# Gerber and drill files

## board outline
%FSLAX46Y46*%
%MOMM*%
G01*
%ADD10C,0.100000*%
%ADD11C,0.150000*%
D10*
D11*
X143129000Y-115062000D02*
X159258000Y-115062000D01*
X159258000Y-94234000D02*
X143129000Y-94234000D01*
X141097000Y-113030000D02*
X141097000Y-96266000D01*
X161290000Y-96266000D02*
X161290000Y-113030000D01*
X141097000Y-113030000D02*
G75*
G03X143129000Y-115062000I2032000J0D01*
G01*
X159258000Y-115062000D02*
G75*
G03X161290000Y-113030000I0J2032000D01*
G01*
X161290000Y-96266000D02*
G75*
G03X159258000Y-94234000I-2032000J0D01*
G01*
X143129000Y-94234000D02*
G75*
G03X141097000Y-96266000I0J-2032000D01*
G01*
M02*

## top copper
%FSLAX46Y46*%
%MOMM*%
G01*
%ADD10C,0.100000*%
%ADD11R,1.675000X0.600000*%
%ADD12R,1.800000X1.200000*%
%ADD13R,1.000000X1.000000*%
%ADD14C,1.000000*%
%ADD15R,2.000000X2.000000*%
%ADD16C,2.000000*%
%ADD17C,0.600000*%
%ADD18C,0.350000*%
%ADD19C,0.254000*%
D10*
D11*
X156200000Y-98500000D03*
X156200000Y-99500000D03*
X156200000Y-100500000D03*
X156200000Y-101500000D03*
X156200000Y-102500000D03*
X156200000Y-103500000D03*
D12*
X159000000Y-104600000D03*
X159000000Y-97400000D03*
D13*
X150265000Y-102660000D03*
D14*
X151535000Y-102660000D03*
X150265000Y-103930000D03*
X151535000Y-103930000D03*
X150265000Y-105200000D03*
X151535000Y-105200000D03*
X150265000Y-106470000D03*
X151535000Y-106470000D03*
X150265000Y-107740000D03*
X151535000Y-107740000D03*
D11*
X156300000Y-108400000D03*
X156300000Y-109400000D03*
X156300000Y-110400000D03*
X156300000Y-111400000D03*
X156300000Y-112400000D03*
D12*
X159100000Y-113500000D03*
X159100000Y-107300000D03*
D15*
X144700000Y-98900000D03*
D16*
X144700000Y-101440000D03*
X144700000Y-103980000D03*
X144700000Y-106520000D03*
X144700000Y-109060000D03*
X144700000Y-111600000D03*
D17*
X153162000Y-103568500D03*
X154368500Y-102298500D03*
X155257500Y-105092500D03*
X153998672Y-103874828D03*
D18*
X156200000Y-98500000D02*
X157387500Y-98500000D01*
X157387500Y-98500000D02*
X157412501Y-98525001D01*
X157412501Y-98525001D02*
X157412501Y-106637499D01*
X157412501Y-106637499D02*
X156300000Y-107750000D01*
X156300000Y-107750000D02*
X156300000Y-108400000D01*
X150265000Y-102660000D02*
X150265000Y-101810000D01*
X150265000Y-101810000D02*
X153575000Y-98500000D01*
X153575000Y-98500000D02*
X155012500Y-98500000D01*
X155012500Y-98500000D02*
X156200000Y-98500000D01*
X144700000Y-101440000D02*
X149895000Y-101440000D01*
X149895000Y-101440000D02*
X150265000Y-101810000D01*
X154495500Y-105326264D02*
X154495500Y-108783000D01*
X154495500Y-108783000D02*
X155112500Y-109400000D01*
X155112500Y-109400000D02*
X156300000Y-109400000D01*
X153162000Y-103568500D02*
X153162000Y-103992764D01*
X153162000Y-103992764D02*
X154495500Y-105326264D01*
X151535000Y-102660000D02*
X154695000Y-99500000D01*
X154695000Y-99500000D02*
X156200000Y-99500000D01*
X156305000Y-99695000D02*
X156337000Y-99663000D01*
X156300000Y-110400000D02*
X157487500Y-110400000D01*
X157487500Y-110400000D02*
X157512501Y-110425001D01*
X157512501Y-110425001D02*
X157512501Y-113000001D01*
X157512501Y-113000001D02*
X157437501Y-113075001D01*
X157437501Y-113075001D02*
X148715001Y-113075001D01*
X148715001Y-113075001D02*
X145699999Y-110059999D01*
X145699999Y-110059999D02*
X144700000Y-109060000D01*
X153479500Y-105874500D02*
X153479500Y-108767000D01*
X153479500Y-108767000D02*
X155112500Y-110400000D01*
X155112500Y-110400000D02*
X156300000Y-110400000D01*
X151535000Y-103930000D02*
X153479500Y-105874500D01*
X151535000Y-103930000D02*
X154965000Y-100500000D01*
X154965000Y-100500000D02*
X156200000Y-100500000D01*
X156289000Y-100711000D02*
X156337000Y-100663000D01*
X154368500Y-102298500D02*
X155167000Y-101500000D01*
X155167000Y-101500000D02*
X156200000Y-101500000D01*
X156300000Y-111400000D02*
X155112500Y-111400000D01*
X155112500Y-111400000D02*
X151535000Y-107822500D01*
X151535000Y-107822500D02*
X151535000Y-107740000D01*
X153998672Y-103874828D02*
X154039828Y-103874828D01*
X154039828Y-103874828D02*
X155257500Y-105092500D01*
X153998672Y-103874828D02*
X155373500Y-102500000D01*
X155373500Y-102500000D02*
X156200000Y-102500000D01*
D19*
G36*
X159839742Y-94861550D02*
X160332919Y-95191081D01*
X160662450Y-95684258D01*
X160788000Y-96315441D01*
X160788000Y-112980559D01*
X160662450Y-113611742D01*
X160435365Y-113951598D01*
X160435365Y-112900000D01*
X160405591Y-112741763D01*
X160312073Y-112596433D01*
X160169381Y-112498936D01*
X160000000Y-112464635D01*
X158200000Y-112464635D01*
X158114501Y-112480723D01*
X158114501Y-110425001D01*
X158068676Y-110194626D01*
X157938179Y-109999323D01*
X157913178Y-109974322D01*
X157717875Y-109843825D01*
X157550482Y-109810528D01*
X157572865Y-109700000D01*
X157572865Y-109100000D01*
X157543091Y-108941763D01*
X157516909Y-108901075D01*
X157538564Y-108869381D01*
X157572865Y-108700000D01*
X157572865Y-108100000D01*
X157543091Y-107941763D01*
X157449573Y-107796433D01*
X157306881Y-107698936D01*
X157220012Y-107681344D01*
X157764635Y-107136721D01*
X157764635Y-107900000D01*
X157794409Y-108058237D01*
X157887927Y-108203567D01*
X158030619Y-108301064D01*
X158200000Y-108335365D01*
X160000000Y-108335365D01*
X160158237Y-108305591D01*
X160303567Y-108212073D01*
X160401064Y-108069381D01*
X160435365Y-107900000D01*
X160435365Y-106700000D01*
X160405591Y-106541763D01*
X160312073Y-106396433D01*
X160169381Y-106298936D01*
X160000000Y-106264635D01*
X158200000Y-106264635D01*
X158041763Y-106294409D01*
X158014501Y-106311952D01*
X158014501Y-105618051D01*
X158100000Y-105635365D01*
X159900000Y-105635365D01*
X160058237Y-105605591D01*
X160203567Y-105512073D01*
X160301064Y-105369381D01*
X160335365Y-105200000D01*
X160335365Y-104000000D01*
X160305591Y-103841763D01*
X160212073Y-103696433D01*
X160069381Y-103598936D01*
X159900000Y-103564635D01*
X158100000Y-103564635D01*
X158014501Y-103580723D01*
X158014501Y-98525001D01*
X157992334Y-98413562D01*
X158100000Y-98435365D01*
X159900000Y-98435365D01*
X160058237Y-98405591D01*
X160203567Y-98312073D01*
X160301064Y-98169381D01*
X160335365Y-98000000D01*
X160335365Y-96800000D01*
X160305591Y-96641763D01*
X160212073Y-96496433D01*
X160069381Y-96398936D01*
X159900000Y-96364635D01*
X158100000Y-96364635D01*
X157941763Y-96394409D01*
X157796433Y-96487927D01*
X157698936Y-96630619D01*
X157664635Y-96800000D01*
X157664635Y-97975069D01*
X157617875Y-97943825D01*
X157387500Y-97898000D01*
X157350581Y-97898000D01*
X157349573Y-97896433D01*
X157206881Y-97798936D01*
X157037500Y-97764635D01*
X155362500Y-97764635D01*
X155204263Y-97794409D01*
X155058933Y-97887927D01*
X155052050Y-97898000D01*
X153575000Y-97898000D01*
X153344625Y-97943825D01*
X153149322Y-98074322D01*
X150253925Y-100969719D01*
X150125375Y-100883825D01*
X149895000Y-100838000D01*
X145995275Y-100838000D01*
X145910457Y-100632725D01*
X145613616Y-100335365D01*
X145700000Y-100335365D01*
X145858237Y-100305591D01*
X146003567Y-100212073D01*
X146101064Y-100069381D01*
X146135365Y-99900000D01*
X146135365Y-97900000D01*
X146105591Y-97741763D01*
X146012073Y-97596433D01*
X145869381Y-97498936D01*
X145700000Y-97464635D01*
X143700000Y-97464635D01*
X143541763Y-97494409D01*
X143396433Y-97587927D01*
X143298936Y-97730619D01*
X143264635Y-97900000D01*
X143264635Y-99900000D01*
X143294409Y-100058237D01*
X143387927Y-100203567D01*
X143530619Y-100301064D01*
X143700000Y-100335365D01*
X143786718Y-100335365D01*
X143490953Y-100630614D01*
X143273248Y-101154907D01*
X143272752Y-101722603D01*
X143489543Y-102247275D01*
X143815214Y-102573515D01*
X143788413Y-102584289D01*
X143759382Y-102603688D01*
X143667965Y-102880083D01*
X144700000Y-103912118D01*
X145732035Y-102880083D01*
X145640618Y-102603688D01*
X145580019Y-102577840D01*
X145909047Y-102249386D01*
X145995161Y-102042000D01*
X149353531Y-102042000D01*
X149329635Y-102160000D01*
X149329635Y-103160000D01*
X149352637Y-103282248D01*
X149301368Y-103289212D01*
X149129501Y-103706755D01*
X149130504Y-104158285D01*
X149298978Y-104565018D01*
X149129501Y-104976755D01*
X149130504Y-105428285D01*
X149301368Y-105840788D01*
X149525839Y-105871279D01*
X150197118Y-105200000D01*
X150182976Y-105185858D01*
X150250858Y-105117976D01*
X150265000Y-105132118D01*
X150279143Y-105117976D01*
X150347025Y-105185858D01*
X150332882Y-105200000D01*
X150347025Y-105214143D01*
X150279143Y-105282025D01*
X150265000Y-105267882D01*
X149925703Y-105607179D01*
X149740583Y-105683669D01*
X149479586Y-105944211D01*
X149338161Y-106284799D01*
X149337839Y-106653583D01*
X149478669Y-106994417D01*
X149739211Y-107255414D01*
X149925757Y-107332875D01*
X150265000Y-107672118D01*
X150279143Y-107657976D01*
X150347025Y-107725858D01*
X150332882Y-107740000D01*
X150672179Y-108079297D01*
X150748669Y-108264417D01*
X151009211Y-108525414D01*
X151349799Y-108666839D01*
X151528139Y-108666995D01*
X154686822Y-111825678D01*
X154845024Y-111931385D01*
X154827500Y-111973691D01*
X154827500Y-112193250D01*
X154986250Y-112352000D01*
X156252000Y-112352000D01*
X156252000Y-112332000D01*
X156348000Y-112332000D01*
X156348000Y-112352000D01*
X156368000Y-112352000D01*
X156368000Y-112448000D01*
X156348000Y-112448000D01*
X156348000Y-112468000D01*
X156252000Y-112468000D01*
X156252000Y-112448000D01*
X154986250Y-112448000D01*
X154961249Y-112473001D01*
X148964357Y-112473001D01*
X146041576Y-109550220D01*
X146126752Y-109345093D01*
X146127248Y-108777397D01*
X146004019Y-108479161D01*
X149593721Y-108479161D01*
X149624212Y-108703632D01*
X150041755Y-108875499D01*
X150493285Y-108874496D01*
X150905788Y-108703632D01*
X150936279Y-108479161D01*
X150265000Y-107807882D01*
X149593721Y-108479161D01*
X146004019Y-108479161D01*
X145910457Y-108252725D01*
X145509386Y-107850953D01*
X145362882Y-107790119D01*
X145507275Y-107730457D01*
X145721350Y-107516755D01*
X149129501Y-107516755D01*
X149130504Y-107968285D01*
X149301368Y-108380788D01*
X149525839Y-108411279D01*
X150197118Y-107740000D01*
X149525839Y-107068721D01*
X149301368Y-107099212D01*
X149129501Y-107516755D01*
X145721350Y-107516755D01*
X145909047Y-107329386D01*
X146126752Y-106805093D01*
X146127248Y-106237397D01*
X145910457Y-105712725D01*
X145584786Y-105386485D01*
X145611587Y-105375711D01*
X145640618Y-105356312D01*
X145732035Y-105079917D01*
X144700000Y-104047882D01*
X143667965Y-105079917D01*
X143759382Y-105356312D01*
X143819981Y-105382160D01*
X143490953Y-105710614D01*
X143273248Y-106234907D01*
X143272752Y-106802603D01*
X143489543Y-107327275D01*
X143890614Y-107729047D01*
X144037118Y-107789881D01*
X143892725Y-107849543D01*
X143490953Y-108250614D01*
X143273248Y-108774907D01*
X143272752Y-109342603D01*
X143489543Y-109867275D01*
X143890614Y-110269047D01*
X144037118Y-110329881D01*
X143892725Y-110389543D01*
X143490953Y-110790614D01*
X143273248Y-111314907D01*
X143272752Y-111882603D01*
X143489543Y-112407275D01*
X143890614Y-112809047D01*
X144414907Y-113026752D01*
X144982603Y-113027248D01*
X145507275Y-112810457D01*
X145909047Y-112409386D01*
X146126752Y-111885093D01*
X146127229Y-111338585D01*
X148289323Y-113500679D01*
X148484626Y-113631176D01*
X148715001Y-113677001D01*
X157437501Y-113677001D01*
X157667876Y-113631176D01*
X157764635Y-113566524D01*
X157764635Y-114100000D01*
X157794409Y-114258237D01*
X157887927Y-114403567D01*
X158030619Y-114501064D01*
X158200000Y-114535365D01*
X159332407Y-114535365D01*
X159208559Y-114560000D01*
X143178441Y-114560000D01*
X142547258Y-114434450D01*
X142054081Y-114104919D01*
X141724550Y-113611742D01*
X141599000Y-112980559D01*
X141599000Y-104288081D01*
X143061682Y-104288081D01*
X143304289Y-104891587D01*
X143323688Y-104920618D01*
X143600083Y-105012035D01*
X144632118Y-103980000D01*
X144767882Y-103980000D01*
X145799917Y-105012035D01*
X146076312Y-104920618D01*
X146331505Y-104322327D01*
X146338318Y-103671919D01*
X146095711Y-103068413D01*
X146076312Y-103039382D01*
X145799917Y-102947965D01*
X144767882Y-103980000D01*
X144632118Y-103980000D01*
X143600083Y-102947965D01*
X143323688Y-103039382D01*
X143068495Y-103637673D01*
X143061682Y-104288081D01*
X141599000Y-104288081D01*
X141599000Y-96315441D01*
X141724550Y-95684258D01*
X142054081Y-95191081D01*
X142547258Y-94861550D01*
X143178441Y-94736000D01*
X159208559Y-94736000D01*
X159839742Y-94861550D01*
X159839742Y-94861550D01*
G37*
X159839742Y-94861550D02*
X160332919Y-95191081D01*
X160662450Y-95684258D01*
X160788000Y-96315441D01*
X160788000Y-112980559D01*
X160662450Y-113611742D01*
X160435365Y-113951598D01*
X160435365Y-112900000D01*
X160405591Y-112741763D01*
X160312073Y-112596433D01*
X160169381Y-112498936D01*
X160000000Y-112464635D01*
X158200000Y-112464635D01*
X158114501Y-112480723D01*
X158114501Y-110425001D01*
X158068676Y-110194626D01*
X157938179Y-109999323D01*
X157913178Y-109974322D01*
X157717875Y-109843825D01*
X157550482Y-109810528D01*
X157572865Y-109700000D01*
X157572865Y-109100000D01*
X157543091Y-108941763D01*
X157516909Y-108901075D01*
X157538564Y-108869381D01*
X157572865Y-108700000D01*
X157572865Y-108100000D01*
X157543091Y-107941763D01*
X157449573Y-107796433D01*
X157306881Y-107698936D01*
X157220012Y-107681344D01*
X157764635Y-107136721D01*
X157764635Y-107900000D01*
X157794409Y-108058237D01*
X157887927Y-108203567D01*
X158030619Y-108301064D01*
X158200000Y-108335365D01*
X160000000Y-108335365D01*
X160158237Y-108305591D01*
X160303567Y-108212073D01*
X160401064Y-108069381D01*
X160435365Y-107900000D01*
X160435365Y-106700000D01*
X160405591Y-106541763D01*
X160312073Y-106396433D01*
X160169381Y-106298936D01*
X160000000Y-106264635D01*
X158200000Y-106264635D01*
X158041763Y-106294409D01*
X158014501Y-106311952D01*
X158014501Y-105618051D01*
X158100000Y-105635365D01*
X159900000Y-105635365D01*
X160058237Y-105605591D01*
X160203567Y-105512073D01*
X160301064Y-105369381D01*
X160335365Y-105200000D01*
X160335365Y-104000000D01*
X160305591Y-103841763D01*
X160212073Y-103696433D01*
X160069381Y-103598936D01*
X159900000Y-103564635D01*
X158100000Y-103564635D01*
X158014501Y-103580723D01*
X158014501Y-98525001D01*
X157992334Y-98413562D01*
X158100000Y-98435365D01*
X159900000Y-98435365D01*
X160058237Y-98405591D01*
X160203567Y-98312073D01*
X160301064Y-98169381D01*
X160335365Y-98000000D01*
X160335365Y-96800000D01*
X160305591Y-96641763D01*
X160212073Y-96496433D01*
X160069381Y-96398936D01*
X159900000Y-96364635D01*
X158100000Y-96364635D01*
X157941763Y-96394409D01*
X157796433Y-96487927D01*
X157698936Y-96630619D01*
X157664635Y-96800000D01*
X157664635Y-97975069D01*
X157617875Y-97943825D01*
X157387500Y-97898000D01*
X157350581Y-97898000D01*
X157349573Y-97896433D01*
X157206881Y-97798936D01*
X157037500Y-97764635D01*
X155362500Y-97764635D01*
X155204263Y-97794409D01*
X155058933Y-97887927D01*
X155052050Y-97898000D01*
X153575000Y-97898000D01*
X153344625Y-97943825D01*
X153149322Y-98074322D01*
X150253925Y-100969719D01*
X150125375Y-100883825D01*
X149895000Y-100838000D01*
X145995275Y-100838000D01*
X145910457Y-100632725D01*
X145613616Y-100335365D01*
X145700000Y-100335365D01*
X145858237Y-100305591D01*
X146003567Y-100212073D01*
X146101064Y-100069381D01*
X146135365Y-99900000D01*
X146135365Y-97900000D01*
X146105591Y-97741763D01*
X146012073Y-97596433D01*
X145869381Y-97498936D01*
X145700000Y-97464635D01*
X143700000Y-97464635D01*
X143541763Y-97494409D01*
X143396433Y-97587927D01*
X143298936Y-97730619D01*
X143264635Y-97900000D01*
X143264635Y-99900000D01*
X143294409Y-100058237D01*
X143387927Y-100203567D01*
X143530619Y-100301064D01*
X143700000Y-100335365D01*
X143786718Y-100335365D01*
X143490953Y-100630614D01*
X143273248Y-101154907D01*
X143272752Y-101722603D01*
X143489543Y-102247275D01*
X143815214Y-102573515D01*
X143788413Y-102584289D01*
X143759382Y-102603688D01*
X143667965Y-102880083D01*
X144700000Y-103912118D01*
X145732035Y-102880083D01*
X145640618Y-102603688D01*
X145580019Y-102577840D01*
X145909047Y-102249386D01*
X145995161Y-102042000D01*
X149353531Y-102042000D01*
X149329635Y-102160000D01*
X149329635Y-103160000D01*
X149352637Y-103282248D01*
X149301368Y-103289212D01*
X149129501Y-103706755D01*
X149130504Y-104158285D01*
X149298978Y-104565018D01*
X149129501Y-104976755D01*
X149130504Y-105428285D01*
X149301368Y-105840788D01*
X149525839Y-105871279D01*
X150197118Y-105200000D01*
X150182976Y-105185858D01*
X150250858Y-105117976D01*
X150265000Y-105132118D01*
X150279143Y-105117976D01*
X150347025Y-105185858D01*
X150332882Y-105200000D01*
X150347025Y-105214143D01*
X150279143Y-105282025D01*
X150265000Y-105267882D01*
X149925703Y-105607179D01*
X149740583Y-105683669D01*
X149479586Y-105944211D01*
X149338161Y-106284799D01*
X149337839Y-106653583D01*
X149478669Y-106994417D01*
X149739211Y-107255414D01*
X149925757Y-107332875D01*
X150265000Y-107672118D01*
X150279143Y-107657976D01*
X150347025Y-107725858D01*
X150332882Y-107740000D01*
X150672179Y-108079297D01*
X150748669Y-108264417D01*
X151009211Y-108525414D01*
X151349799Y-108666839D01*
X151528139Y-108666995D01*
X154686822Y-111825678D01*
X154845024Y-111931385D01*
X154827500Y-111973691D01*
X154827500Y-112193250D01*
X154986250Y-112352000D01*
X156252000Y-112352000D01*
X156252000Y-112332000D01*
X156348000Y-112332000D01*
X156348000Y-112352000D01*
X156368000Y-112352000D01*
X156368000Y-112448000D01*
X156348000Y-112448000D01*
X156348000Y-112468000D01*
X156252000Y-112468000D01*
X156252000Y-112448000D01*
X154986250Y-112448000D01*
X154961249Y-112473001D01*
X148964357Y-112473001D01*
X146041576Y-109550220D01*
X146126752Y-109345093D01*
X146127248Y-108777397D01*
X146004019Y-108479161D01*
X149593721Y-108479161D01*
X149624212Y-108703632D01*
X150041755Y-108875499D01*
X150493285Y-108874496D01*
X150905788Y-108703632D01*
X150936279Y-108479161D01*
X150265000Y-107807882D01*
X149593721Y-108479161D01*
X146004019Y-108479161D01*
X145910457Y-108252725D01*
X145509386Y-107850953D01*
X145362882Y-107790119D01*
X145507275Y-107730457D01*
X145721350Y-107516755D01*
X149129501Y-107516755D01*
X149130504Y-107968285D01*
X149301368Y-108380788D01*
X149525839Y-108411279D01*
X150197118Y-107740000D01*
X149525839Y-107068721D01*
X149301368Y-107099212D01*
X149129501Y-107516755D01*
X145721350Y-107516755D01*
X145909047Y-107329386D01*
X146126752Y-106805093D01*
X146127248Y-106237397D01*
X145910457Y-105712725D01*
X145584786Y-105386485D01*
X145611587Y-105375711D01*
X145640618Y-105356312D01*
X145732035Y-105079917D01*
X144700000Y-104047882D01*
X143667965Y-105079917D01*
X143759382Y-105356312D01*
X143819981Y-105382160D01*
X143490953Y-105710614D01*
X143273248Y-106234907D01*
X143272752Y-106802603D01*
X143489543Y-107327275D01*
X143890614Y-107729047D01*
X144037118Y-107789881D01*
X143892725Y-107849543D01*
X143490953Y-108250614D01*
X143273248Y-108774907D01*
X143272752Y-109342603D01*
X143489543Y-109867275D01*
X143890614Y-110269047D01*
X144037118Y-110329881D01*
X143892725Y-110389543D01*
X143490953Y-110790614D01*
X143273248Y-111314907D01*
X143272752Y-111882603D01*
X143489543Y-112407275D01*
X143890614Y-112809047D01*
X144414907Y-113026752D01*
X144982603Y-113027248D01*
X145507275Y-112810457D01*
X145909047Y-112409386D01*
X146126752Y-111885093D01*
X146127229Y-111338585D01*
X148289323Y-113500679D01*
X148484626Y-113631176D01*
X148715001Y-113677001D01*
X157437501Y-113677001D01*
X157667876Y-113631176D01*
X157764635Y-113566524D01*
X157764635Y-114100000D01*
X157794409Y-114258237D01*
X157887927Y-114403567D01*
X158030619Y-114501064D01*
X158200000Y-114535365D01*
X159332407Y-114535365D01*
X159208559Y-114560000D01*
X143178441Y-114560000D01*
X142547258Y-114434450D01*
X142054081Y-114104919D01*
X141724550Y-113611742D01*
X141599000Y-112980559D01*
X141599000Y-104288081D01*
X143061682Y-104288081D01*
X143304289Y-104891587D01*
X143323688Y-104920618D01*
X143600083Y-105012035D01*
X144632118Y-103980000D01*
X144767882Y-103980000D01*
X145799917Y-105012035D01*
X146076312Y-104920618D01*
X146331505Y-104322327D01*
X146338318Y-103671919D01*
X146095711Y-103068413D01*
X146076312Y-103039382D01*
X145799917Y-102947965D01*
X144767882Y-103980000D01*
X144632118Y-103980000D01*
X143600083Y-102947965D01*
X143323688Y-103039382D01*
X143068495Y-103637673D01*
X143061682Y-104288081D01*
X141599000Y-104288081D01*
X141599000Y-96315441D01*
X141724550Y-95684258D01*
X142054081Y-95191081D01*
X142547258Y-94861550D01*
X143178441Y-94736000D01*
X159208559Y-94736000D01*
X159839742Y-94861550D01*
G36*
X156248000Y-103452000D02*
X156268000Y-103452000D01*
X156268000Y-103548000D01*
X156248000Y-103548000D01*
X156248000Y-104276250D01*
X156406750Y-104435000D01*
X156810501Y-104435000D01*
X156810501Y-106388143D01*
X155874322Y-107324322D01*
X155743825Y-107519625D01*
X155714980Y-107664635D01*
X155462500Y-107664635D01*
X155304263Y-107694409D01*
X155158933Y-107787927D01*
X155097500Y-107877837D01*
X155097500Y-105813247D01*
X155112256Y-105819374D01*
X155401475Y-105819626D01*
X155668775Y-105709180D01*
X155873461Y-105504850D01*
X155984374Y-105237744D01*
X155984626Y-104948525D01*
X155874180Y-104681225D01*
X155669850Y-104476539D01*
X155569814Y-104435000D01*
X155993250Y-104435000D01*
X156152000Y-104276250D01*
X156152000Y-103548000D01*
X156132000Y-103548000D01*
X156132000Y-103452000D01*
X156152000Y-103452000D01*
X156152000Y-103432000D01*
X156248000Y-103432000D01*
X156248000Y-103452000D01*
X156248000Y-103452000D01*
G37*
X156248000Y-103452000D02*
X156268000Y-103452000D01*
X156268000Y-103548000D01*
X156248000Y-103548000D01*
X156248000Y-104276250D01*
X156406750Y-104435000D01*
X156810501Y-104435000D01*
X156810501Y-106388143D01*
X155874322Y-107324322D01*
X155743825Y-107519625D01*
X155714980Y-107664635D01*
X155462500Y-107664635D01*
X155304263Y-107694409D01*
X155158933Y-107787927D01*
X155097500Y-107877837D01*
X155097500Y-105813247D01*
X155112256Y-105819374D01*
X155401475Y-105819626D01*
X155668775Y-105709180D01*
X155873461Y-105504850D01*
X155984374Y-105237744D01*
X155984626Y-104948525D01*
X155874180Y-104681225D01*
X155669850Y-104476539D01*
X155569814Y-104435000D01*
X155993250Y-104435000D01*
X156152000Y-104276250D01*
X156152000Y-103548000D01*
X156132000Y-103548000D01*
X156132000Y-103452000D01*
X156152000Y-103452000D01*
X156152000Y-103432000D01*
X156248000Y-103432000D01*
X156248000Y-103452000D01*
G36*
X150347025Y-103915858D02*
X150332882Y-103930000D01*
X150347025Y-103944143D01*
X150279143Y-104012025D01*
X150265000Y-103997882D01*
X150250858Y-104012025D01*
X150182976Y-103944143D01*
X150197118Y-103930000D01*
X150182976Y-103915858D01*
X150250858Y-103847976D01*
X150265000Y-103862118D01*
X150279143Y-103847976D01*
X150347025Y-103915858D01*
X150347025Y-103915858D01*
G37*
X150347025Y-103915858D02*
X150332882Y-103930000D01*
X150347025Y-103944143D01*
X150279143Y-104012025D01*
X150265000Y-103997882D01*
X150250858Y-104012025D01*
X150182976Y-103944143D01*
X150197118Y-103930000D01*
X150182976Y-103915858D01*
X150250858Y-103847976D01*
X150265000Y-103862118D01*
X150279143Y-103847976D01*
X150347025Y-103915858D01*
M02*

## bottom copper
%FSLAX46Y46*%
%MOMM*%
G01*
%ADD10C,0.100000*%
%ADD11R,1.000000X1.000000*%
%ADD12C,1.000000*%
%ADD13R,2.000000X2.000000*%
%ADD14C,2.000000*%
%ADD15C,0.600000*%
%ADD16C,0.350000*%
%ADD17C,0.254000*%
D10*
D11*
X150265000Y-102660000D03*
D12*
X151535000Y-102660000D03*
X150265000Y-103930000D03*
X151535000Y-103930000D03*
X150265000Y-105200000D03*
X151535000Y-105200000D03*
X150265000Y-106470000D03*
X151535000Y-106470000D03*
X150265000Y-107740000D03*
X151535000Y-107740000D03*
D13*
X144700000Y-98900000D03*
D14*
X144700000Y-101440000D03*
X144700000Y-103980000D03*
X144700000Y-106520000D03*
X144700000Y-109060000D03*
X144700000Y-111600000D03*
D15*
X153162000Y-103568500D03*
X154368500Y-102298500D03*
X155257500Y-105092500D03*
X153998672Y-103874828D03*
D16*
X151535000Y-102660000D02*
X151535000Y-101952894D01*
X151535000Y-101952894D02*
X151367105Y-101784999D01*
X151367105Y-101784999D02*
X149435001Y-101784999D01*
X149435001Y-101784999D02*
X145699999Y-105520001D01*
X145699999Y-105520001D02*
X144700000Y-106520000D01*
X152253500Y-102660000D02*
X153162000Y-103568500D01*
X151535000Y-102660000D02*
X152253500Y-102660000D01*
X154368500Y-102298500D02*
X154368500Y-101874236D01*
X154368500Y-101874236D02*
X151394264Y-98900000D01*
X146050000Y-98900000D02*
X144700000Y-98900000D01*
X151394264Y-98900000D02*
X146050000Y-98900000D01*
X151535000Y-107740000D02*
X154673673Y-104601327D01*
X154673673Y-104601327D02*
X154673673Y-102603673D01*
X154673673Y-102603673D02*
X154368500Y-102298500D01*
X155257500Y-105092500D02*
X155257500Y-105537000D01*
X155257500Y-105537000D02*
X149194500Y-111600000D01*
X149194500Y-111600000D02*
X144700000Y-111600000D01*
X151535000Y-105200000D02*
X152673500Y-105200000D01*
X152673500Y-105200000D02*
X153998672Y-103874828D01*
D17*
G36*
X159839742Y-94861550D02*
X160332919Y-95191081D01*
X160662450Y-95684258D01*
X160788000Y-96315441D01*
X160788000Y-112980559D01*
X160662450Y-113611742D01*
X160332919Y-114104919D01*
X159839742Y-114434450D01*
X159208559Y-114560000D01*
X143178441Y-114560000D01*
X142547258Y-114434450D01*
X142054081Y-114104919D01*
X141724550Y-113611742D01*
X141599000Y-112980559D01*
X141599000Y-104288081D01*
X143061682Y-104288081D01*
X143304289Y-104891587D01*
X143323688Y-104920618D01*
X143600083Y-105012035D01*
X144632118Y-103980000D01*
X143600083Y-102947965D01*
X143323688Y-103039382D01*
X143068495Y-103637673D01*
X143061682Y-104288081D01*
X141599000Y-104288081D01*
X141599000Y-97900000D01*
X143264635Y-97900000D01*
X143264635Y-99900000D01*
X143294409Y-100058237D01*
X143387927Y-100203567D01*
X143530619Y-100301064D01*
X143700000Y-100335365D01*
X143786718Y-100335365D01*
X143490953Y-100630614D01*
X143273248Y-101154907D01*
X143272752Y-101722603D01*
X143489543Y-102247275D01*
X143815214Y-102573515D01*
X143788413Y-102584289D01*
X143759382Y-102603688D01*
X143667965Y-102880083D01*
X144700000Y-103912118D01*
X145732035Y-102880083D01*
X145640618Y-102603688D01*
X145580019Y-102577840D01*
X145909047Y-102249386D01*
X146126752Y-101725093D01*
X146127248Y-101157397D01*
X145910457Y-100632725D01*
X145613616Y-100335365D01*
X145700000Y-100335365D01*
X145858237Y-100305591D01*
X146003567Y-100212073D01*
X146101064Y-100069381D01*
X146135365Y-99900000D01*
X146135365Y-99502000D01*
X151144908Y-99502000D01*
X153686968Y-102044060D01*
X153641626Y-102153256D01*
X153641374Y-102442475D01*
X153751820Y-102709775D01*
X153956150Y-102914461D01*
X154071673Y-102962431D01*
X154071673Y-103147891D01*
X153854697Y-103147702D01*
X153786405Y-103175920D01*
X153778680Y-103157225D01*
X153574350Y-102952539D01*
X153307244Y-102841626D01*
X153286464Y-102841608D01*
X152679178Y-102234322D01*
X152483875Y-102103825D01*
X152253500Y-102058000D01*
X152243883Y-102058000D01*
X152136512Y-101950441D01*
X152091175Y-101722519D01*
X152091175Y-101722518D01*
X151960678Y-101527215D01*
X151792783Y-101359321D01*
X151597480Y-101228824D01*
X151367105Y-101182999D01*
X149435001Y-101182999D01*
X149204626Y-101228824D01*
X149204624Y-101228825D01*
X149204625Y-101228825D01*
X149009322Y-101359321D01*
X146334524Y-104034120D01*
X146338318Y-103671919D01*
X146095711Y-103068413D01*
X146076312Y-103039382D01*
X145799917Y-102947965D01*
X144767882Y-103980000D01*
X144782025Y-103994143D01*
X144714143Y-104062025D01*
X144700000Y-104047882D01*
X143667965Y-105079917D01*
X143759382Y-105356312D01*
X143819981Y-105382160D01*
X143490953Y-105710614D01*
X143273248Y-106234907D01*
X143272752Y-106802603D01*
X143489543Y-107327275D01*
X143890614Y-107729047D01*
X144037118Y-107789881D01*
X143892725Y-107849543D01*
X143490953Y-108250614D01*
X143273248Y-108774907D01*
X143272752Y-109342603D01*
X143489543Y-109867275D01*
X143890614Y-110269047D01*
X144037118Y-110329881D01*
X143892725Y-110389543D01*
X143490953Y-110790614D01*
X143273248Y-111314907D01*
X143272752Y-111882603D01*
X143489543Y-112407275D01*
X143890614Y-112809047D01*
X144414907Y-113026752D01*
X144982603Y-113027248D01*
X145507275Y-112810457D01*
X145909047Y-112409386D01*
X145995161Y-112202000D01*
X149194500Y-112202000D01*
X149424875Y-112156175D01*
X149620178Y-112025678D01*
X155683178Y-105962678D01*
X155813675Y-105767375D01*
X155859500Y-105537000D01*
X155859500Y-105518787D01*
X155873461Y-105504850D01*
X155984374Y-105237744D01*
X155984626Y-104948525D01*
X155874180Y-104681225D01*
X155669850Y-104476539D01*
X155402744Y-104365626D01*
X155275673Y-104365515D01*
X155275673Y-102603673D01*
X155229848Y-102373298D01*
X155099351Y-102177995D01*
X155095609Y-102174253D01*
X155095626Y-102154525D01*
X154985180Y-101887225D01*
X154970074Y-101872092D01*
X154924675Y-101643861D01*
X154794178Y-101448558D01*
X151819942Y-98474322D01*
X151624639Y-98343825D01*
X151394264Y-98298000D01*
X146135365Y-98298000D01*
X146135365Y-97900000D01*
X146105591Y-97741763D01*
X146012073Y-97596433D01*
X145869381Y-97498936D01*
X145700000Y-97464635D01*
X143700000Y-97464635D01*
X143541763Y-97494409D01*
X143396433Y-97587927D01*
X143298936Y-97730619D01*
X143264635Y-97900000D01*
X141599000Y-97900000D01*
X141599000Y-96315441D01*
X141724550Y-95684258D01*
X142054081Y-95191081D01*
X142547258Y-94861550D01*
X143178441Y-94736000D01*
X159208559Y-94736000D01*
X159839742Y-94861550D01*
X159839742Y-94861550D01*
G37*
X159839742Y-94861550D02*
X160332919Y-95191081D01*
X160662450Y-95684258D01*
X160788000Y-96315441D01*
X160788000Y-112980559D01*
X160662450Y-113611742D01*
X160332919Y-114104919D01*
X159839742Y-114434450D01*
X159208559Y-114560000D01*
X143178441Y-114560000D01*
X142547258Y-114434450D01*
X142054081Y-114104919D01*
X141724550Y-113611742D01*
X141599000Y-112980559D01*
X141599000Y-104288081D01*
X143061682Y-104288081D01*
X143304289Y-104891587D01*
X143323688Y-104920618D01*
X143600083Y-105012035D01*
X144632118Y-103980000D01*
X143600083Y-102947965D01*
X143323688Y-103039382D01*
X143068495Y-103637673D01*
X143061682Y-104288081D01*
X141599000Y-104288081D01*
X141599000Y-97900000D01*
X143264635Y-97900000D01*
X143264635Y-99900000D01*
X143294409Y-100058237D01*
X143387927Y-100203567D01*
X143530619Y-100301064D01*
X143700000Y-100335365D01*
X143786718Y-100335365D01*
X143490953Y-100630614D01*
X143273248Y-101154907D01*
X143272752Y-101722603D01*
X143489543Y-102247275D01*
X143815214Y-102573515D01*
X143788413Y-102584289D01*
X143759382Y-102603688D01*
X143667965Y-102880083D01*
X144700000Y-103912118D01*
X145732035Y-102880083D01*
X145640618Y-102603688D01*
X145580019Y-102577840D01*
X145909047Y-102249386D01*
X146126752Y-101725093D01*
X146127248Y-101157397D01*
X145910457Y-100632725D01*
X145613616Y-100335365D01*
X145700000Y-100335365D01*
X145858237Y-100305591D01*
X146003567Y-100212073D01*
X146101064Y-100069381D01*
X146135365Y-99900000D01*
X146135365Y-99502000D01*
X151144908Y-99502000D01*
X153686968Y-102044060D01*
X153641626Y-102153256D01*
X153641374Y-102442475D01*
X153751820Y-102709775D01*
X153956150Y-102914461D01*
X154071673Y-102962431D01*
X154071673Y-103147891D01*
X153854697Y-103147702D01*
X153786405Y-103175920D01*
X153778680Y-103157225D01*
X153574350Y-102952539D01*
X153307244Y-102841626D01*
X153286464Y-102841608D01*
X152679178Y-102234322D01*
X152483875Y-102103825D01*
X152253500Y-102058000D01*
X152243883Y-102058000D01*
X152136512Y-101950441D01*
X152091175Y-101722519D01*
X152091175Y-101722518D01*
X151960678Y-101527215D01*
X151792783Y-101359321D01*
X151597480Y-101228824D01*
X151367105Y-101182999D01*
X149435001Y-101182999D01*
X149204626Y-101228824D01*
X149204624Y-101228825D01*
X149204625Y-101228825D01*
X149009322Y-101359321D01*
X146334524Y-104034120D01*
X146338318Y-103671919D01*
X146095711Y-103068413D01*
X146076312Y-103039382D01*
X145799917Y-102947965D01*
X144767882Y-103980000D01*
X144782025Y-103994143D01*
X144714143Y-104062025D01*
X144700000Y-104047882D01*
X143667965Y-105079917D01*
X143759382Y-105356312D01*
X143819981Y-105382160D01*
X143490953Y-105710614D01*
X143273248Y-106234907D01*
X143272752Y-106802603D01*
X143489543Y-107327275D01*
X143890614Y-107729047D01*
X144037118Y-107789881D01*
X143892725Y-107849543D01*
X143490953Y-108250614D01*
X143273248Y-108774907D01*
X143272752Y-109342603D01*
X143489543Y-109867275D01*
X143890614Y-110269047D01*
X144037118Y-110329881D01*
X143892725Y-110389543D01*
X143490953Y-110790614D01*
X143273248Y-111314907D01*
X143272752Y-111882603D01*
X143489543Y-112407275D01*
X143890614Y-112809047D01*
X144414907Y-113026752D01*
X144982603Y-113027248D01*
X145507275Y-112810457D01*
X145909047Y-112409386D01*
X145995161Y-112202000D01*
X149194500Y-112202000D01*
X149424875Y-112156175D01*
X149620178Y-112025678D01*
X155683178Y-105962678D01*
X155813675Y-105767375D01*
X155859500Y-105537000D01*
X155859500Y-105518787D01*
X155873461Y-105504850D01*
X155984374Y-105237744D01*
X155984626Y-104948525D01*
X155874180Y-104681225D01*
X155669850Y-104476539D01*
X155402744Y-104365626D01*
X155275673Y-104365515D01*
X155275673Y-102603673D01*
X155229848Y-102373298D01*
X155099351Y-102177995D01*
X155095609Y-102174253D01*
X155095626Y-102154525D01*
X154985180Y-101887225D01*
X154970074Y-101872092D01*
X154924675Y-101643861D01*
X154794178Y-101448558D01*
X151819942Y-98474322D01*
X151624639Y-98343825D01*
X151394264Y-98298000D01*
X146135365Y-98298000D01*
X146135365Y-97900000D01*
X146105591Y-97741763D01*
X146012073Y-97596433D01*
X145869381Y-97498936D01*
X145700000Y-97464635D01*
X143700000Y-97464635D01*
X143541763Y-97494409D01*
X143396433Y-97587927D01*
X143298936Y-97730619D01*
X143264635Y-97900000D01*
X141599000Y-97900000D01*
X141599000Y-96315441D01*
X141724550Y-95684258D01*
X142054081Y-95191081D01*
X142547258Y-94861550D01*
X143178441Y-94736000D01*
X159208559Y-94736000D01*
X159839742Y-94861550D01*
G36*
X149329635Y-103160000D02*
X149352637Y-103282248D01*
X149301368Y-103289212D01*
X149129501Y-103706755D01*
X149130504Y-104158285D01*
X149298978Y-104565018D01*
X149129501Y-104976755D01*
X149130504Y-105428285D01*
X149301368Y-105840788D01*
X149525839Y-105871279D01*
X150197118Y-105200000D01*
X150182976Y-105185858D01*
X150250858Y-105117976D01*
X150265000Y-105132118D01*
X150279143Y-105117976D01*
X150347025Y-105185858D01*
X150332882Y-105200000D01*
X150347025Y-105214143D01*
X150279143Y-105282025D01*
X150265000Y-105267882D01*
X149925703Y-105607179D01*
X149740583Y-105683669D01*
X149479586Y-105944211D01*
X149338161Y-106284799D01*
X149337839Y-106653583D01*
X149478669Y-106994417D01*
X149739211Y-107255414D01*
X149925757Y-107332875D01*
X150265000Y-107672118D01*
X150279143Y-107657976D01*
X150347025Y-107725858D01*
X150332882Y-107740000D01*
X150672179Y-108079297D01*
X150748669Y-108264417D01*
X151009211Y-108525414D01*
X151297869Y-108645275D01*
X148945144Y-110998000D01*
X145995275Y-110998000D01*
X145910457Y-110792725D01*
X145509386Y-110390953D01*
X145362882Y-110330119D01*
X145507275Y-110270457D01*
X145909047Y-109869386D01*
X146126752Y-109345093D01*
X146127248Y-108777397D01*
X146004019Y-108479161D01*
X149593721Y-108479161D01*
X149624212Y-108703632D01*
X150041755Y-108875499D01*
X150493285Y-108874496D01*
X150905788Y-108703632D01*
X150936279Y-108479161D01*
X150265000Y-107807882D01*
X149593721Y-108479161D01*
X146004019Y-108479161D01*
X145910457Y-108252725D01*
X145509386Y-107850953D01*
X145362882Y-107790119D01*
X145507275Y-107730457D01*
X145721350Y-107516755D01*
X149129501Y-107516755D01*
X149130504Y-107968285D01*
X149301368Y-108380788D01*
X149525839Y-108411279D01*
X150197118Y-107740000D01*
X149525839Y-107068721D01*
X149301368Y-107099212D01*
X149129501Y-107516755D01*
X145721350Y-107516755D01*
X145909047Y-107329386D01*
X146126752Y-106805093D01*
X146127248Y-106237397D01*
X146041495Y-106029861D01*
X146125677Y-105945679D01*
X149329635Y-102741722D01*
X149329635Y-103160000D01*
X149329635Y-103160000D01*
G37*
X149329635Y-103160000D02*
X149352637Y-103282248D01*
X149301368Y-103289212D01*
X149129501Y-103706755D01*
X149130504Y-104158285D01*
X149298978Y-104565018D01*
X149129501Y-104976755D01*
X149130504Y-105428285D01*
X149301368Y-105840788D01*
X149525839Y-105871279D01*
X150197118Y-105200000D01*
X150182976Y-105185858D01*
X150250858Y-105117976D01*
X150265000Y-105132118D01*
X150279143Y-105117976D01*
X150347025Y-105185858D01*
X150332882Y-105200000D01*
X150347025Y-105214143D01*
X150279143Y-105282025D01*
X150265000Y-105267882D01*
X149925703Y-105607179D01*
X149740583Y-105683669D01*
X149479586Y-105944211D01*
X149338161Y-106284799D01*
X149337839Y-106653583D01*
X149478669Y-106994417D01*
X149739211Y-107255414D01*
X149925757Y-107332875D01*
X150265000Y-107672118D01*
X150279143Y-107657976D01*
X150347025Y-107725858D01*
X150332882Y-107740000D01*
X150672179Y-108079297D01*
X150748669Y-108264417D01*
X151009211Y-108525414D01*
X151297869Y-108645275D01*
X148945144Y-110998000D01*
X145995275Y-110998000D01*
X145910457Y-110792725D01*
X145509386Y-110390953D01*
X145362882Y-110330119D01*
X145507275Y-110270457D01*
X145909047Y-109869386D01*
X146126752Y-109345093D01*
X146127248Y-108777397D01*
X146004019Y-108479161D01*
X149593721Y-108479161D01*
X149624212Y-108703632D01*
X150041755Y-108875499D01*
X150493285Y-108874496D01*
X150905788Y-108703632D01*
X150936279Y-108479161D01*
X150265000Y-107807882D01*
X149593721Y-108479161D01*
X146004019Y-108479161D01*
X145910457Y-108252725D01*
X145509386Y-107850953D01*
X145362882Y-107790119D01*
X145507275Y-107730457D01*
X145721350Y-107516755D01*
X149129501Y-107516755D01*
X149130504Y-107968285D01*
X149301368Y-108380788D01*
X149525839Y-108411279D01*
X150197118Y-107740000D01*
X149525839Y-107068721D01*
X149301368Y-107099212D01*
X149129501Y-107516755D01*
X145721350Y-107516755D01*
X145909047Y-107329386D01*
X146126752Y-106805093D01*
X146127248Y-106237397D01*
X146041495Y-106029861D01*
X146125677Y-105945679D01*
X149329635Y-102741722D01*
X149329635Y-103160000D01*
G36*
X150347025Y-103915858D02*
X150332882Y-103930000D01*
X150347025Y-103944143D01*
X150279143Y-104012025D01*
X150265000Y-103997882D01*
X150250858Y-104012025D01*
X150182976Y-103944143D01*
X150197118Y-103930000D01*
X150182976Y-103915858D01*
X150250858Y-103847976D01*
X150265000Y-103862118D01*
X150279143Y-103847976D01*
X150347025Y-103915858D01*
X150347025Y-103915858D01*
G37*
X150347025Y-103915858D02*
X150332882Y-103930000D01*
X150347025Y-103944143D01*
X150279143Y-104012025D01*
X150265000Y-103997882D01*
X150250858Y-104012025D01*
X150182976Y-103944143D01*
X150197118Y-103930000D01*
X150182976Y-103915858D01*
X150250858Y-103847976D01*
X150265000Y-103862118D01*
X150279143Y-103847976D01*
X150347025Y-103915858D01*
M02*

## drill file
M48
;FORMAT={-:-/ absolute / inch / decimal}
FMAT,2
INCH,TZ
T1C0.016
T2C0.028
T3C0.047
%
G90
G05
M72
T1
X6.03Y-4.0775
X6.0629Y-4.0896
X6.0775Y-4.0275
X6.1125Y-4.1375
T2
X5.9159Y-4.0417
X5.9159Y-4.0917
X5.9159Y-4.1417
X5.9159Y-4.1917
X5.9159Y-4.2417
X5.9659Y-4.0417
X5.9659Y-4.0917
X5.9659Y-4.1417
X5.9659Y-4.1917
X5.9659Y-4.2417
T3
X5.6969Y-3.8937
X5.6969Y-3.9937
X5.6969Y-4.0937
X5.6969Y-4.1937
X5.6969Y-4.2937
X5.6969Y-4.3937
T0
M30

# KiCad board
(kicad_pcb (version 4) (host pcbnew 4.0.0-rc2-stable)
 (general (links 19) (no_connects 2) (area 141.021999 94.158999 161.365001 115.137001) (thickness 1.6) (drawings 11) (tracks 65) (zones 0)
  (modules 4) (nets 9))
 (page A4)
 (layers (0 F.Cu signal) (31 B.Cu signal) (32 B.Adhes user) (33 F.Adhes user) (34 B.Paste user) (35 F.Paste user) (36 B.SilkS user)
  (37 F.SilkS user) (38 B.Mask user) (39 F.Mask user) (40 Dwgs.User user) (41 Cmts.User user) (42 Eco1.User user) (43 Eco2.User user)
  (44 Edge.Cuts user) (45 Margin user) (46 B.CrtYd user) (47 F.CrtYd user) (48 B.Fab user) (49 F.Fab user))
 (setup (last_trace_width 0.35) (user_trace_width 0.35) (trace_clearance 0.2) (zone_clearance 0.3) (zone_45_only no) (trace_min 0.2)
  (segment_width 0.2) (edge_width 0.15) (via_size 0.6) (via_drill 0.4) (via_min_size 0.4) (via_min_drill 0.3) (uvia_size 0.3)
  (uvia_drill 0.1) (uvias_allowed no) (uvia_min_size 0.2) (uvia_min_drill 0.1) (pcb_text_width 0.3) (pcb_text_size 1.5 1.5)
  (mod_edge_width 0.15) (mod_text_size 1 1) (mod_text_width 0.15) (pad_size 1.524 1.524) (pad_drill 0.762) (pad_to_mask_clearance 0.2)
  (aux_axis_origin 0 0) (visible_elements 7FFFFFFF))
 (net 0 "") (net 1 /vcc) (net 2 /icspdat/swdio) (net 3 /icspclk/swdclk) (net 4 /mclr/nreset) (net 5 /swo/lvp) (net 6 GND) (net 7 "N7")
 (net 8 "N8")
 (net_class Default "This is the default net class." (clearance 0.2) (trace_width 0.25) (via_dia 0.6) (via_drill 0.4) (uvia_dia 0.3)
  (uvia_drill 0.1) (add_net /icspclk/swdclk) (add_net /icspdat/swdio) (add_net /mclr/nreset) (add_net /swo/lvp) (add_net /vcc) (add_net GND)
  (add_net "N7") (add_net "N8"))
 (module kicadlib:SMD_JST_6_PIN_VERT (layer F.Cu) (at 156.2 98.5 270)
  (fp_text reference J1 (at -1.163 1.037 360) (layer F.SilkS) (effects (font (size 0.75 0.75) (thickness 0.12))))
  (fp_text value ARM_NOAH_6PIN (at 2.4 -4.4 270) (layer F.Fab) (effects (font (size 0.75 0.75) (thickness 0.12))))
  (pad 1 smd rect (at 0 0 270) (size 0.6 1.675) (layers F.Cu F.Paste F.Mask) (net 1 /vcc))
  (pad 2 smd rect (at 1 0 270) (size 0.6 1.675) (layers F.Cu F.Paste F.Mask) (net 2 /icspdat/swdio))
  (pad 3 smd rect (at 2 0 270) (size 0.6 1.675) (layers F.Cu F.Paste F.Mask) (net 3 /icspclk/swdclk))
  (pad 4 smd rect (at 3 0 270) (size 0.6 1.675) (layers F.Cu F.Paste F.Mask) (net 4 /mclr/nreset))
  (pad 5 smd rect (at 4 0 270) (size 0.6 1.675) (layers F.Cu F.Paste F.Mask) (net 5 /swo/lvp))
  (pad 6 smd rect (at 5 0 270) (size 0.6 1.675) (layers F.Cu F.Paste F.Mask) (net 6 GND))
  (pad "" smd rect (at 6.1 -2.8 270) (size 1.2 1.8) (layers F.Cu F.Paste F.Mask))
  (pad "" smd rect (at -1.1 -2.8 270) (size 1.2 1.8) (layers F.Cu F.Paste F.Mask)))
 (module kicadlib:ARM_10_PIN (layer F.Cu) (at 150.9 105.2)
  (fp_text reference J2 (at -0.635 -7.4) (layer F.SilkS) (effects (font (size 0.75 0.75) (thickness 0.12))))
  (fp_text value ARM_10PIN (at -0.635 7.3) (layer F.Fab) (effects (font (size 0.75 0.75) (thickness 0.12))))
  (pad 1 thru_hole rect (at -0.635 -2.54) (size 1 1) (drill 0.70104) (layers *.Cu *.Mask F.SilkS) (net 1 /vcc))
  (pad 2 thru_hole circle (at 0.635 -2.54) (size 1 1) (drill 0.70104) (layers *.Cu *.Mask F.SilkS) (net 2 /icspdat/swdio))
  (pad 3 thru_hole circle (at -0.635 -1.27) (size 1 1) (drill 0.70104) (layers *.Cu *.Mask F.SilkS) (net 6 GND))
  (pad 4 thru_hole circle (at 0.635 -1.27) (size 1 1) (drill 0.70104) (layers *.Cu *.Mask F.SilkS) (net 3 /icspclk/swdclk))
  (pad 5 thru_hole circle (at -0.635 0) (size 1 1) (drill 0.70104) (layers *.Cu *.Mask F.SilkS) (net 6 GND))
  (pad 6 thru_hole circle (at 0.635 0) (size 1 1) (drill 0.70104) (layers *.Cu *.Mask F.SilkS) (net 5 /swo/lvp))
  (pad 7 thru_hole circle (at -0.635 1.27) (size 1 1) (drill 0.70104) (layers *.Cu *.Mask F.SilkS) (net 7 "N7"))
  (pad 8 thru_hole circle (at 0.635 1.27) (size 1 1) (drill 0.70104) (layers *.Cu *.Mask F.SilkS) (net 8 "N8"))
  (pad 9 thru_hole circle (at -0.635 2.54) (size 1 1) (drill 0.70104) (layers *.Cu *.Mask F.SilkS) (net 6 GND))
  (pad 10 thru_hole circle (at 0.635 2.54) (size 1 1) (drill 0.70104) (layers *.Cu *.Mask F.SilkS) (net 4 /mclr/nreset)))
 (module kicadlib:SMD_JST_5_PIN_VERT (layer F.Cu) (at 156.3 108.4 270)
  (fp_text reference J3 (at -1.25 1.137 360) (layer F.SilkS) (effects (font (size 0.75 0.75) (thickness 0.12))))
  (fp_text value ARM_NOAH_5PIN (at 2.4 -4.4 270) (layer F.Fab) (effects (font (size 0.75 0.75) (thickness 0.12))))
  (pad 1 smd rect (at 0 0 270) (size 0.6 1.675) (layers F.Cu F.Paste F.Mask) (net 1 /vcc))
  (pad 2 smd rect (at 1 0 270) (size 0.6 1.675) (layers F.Cu F.Paste F.Mask) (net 2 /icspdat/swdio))
  (pad 3 smd rect (at 2 0 270) (size 0.6 1.675) (layers F.Cu F.Paste F.Mask) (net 3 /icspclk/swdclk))
  (pad 4 smd rect (at 3 0 270) (size 0.6 1.675) (layers F.Cu F.Paste F.Mask) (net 4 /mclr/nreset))
  (pad 5 smd rect (at 4 0 270) (size 0.6 1.675) (layers F.Cu F.Paste F.Mask) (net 6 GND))
  (pad "" smd rect (at 5.1 -2.8 270) (size 1.2 1.8) (layers F.Cu F.Paste F.Mask))
  (pad "" smd rect (at -1.1 -2.8 270) (size 1.2 1.8) (layers F.Cu F.Paste F.Mask)))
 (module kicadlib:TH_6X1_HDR (layer F.Cu) (at 144.7 98.9 270)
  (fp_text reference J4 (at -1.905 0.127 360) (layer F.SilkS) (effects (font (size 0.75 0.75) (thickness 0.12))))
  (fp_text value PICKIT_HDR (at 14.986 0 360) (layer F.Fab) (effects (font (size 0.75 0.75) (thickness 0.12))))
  (pad 1 thru_hole rect (at 0 0 270) (size 2 2) (drill 1.2) (layers *.Cu *.Mask F.SilkS) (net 4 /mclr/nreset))
  (pad 2 thru_hole circle (at 2.54 0 270) (size 2 2) (drill 1.2) (layers *.Cu *.Mask F.SilkS) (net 1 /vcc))
  (pad 3 thru_hole circle (at 5.08 0 270) (size 2 2) (drill 1.2) (layers *.Cu *.Mask F.SilkS) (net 6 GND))
  (pad 4 thru_hole circle (at 7.62 0 270) (size 2 2) (drill 1.2) (layers *.Cu *.Mask F.SilkS) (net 2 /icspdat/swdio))
  (pad 5 thru_hole circle (at 10.16 0 270) (size 2 2) (drill 1.2) (layers *.Cu *.Mask F.SilkS) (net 3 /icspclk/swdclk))
  (pad 6 thru_hole circle (at 12.7 0 270) (size 2 2) (drill 1.2) (layers *.Cu *.Mask F.SilkS) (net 5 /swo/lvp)))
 (gr_line (start 143.129 115.062) (end 159.258 115.062) (angle 90) (layer Edge.Cuts) (width 0.15))
 (gr_line (start 159.258 94.234) (end 143.129 94.234) (angle 90) (layer Edge.Cuts) (width 0.15))
 (gr_line (start 141.097 113.03) (end 141.097 96.266) (angle 90) (layer Edge.Cuts) (width 0.15))
 (gr_line (start 161.29 96.266) (end 161.29 113.03) (angle 90) (layer Edge.Cuts) (width 0.15))
 (gr_arc (start 143.129 113.03) (end 143.129 115.062) (angle 90) (layer Edge.Cuts) (width 0.15))
 (gr_arc (start 159.258 113.03) (end 161.29 113.03) (angle 90) (layer Edge.Cuts) (width 0.15))
 (gr_arc (start 159.258 96.266) (end 159.258 94.234) (angle 90) (layer Edge.Cuts) (width 0.15))
 (gr_arc (start 143.129 96.266) (end 141.097 96.266) (angle 90) (layer Edge.Cuts) (width 0.15))
 (segment (start 156.2 98.5) (end 157.3875 98.5) (width 0.35) (layer F.Cu) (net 1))
 (segment (start 157.3875 98.5) (end 157.412501 98.525001) (width 0.35) (layer F.Cu) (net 1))
 (segment (start 157.412501 98.525001) (end 157.412501 106.637499) (width 0.35) (layer F.Cu) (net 1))
 (segment (start 157.412501 106.637499) (end 156.3 107.75) (width 0.35) (layer F.Cu) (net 1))
 (segment (start 156.3 107.75) (end 156.3 108.4) (width 0.35) (layer F.Cu) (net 1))
 (segment (start 150.265 102.66) (end 150.265 101.81) (width 0.35) (layer F.Cu) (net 1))
 (segment (start 150.265 101.81) (end 153.575 98.5) (width 0.35) (layer F.Cu) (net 1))
 (segment (start 153.575 98.5) (end 155.0125 98.5) (width 0.35) (layer F.Cu) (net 1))
 (segment (start 155.0125 98.5) (end 156.2 98.5) (width 0.35) (layer F.Cu) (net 1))
 (segment (start 144.7 101.44) (end 149.895 101.44) (width 0.35) (layer F.Cu) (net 1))
 (segment (start 149.895 101.44) (end 150.265 101.81) (width 0.35) (layer F.Cu) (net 1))
 (segment (start 151.535 102.66) (end 151.535 101.952894) (width 0.35) (layer B.Cu) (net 2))
 (segment (start 151.535 101.952894) (end 151.367105 101.784999) (width 0.35) (layer B.Cu) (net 2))
 (segment (start 151.367105 101.784999) (end 149.435001 101.784999) (width 0.35) (layer B.Cu) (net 2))
 (segment (start 149.435001 101.784999) (end 145.699999 105.520001) (width 0.35) (layer B.Cu) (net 2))
 (segment (start 145.699999 105.520001) (end 144.7 106.52) (width 0.35) (layer B.Cu) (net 2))
 (segment (start 154.4955 105.326264) (end 154.4955 108.783) (width 0.35) (layer F.Cu) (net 2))
 (segment (start 154.4955 108.783) (end 155.1125 109.4) (width 0.35) (layer F.Cu) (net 2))
 (segment (start 155.1125 109.4) (end 156.3 109.4) (width 0.35) (layer F.Cu) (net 2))
 (segment (start 153.162 103.5685) (end 153.162 103.992764) (width 0.35) (layer F.Cu) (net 2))
 (segment (start 153.162 103.992764) (end 154.4955 105.326264) (width 0.35) (layer F.Cu) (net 2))
 (segment (start 152.2535 102.66) (end 153.162 103.5685) (width 0.35) (layer B.Cu) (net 2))
 (via (at 153.162 103.5685) (size 0.6) (drill 0.4) (layers F.Cu B.Cu) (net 2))
 (segment (start 151.535 102.66) (end 152.2535 102.66) (width 0.35) (layer B.Cu) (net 2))
 (segment (start 151.535 102.66) (end 154.695 99.5) (width 0.35) (layer F.Cu) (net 2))
 (segment (start 154.695 99.5) (end 156.2 99.5) (width 0.35) (layer F.Cu) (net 2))
 (segment (start 156.305 99.695) (end 156.337 99.663) (width 0.35) (layer F.Cu) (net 2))
 (segment (start 156.3 110.4) (end 157.4875 110.4) (width 0.35) (layer F.Cu) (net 3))
 (segment (start 157.4875 110.4) (end 157.512501 110.425001) (width 0.35) (layer F.Cu) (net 3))
 (segment (start 157.512501 110.425001) (end 157.512501 113.000001) (width 0.35) (layer F.Cu) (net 3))
 (segment (start 157.512501 113.000001) (end 157.437501 113.075001) (width 0.35) (layer F.Cu) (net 3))
 (segment (start 157.437501 113.075001) (end 148.715001 113.075001) (width 0.35) (layer F.Cu) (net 3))
 (segment (start 148.715001 113.075001) (end 145.699999 110.059999) (width 0.35) (layer F.Cu) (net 3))
 (segment (start 145.699999 110.059999) (end 144.7 109.06) (width 0.35) (layer F.Cu) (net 3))
 (segment (start 153.4795 105.8745) (end 153.4795 108.767) (width 0.35) (layer F.Cu) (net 3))
 (segment (start 153.4795 108.767) (end 155.1125 110.4) (width 0.35) (layer F.Cu) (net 3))
 (segment (start 155.1125 110.4) (end 156.3 110.4) (width 0.35) (layer F.Cu) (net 3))
 (segment (start 151.535 103.93) (end 153.4795 105.8745) (width 0.35) (layer F.Cu) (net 3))
 (segment (start 151.535 103.93) (end 154.965 100.5) (width 0.35) (layer F.Cu) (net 3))
 (segment (start 154.965 100.5) (end 156.2 100.5) (width 0.35) (layer F.Cu) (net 3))
 (segment (start 156.289 100.711) (end 156.337 100.663) (width 0.35) (layer F.Cu) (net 3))
 (segment (start 154.3685 102.2985) (end 154.3685 101.874236) (width 0.35) (layer B.Cu) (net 4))
 (segment (start 154.3685 101.874236) (end 151.394264 98.9) (width 0.35) (layer B.Cu) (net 4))
 (segment (start 146.05 98.9) (end 144.7 98.9) (width 0.35) (layer B.Cu) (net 4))
 (segment (start 151.394264 98.9) (end 146.05 98.9) (width 0.35) (layer B.Cu) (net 4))
 (segment (start 154.3685 102.2985) (end 155.167 101.5) (width 0.35) (layer F.Cu) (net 4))
 (segment (start 155.167 101.5) (end 156.2 101.5) (width 0.35) (layer F.Cu) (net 4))
 (segment (start 151.535 107.74) (end 154.673673 104.601327) (width 0.35) (layer B.Cu) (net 4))
 (segment (start 154.673673 104.601327) (end 154.673673 102.603673) (width 0.35) (layer B.Cu) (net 4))
 (segment (start 154.673673 102.603673) (end 154.3685 102.2985) (width 0.35) (layer B.Cu) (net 4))
 (via (at 154.3685 102.2985) (size 0.6) (drill 0.4) (layers F.Cu B.Cu) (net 4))
 (segment (start 156.3 111.4) (end 155.1125 111.4) (width 0.35) (layer F.Cu) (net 4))
 (segment (start 155.1125 111.4) (end 151.535 107.8225) (width 0.35) (layer F.Cu) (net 4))
 (segment (start 151.535 107.8225) (end 151.535 107.74) (width 0.35) (layer F.Cu) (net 4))
 (segment (start 155.2575 105.0925) (end 155.2575 105.537) (width 0.35) (layer B.Cu) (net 5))
 (segment (start 155.2575 105.537) (end 149.1945 111.6) (width 0.35) (layer B.Cu) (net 5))
 (segment (start 149.1945 111.6) (end 144.7 111.6) (width 0.35) (layer B.Cu) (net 5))
 (segment (start 153.998672 103.874828) (end 154.039828 103.874828) (width 0.35) (layer F.Cu) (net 5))
 (segment (start 154.039828 103.874828) (end 155.2575 105.0925) (width 0.35) (layer F.Cu) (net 5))
 (via (at 155.2575 105.0925) (size 0.6) (drill 0.4) (layers F.Cu B.Cu) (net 5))
 (segment (start 153.998672 103.874828) (end 155.3735 102.5) (width 0.35) (layer F.Cu) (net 5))
 (segment (start 155.3735 102.5) (end 156.2 102.5) (width 0.35) (layer F.Cu) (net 5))
 (segment (start 151.535 105.2) (end 152.6735 105.2) (width 0.35) (layer B.Cu) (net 5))
 (segment (start 152.6735 105.2) (end 153.998672 103.874828) (width 0.35) (layer B.Cu) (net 5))
 (via (at 153.998672 103.874828) (size 0.6) (drill 0.4) (layers F.Cu B.Cu) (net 5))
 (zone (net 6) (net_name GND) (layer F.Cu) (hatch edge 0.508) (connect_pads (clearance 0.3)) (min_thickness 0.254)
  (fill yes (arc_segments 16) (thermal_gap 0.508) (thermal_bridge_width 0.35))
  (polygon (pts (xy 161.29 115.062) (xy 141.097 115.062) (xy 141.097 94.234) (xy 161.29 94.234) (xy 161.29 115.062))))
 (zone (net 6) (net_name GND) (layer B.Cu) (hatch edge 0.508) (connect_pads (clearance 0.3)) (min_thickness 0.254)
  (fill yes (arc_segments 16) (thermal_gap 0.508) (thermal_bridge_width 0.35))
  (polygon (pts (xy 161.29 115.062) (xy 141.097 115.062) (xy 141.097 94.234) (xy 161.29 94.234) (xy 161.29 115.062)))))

